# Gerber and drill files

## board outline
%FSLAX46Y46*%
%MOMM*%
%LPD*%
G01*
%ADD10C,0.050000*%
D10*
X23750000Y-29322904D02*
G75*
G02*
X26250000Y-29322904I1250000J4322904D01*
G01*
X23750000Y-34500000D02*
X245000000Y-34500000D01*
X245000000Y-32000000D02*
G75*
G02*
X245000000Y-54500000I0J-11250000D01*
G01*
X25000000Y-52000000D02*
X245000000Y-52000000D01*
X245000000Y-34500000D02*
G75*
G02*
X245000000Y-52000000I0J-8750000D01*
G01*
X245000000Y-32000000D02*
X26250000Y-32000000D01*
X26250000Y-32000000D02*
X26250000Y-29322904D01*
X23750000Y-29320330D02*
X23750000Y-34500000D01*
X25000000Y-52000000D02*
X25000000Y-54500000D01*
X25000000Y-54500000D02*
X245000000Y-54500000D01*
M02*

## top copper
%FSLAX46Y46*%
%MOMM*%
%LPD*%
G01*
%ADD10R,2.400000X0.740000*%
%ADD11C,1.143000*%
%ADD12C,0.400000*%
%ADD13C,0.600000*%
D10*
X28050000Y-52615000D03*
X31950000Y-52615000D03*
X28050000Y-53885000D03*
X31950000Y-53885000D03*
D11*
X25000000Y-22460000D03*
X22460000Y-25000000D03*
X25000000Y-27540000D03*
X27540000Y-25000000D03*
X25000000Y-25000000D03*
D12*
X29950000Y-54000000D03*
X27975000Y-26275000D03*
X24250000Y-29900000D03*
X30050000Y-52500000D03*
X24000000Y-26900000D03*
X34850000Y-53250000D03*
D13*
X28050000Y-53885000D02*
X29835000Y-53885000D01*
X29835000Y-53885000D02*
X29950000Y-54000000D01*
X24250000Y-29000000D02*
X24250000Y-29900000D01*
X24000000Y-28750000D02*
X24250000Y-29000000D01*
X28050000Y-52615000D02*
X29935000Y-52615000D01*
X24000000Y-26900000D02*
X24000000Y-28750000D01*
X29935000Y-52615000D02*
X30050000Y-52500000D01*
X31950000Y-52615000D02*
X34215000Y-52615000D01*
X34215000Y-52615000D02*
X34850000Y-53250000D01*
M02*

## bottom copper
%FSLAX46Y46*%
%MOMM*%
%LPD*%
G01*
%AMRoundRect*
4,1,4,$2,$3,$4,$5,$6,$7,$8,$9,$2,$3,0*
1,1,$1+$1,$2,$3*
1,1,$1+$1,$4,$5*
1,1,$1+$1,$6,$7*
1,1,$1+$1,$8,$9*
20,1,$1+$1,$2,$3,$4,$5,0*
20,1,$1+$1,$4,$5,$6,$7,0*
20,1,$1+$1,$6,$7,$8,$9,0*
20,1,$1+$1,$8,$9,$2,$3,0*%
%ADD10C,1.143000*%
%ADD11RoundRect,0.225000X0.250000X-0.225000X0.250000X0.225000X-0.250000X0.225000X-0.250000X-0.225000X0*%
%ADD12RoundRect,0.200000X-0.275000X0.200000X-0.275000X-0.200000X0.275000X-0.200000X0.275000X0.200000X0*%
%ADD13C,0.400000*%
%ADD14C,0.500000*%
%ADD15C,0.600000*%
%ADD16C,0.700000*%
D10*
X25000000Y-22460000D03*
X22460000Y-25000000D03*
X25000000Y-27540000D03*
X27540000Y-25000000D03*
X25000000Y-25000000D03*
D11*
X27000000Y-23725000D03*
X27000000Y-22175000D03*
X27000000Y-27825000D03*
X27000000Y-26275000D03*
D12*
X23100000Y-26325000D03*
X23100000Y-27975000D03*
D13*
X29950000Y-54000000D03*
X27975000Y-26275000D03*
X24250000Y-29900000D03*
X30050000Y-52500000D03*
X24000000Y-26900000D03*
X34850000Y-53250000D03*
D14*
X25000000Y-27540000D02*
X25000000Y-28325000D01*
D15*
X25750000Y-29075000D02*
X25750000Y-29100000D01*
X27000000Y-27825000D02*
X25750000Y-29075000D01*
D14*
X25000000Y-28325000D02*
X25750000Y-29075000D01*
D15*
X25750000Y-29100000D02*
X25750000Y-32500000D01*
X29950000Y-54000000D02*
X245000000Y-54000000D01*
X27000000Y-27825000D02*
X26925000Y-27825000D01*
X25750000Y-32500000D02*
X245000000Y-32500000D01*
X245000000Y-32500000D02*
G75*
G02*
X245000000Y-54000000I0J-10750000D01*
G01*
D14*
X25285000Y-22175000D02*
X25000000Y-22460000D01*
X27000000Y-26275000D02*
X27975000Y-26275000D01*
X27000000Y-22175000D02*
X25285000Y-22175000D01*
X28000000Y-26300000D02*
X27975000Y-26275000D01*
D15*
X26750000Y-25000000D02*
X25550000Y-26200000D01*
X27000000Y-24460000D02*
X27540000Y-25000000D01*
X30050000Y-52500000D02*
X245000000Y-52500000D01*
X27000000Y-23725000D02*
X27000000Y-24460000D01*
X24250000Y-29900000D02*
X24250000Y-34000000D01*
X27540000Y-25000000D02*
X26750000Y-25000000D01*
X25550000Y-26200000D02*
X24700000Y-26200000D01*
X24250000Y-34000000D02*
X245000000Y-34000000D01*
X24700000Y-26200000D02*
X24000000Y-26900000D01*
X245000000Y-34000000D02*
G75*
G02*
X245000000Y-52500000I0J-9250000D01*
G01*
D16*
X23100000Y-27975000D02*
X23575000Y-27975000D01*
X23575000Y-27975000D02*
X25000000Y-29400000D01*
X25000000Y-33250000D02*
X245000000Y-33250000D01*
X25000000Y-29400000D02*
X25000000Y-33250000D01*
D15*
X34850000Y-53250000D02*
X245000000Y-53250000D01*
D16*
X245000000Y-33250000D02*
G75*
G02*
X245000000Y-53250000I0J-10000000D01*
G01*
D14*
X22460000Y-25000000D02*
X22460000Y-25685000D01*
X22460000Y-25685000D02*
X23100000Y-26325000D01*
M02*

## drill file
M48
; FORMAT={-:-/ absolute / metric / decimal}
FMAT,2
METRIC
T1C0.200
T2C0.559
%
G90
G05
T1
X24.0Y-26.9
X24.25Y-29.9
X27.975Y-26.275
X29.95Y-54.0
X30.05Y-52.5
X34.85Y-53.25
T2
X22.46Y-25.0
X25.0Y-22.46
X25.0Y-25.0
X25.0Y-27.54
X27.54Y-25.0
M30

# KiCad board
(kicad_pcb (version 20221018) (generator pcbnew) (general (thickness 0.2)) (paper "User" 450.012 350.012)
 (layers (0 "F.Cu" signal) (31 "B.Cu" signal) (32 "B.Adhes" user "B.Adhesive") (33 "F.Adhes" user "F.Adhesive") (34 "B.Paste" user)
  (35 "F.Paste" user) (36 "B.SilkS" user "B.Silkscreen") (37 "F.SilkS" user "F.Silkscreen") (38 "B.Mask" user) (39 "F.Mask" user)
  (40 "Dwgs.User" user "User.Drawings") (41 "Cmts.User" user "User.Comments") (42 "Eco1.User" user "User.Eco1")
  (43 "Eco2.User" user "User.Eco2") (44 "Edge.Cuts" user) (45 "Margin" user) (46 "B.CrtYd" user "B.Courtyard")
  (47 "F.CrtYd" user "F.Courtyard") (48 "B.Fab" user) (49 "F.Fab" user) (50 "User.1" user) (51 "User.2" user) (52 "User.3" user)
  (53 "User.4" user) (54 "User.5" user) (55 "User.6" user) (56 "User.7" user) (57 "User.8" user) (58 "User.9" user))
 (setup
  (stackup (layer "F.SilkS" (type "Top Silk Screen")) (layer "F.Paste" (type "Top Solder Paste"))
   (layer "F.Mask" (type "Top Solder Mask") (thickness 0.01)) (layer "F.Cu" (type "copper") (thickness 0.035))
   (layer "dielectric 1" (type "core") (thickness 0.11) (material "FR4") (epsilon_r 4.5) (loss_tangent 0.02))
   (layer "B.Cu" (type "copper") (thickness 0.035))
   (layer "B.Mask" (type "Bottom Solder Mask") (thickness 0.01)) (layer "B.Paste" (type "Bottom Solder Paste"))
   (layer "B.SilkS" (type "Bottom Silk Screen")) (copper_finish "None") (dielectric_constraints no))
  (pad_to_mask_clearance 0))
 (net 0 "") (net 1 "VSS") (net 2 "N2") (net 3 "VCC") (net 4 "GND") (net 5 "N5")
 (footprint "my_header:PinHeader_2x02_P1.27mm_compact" (layer "F.Cu") (at 30 53.25)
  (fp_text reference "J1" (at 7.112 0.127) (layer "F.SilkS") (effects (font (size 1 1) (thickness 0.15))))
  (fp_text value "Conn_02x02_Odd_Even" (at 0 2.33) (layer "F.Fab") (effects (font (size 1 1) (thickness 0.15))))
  (pad "1" smd rect (at -1.95 -0.635) (size 2.4 0.74) (layers "F.Cu" "F.Paste" "F.Mask") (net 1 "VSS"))
  (pad "2" smd rect (at 1.95 -0.635) (size 2.4 0.74) (layers "F.Cu" "F.Paste" "F.Mask") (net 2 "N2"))
  (pad "3" smd rect (at -1.95 0.635) (size 2.4 0.74) (layers "F.Cu" "F.Paste" "F.Mask") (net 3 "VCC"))
  (pad "4" smd rect (at 1.95 0.635) (size 2.4 0.74) (layers "F.Cu" "F.Paste" "F.Mask") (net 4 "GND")))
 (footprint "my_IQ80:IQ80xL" (layer "F.Cu") (at 25 25 90)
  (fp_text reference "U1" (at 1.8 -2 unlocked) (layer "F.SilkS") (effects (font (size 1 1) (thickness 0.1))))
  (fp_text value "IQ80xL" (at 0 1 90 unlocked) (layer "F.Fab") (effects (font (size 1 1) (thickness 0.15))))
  (pad "1" thru_hole circle (at 2.54 0 90) (size 1.143 1.143) (drill 0.5588) (layers "*.Cu" "*.Mask") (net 4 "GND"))
  (pad "2" thru_hole circle (at 0 -2.54 90) (size 1.143 1.143) (drill 0.5588) (layers "*.Cu" "*.Mask") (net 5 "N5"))
  (pad "3" thru_hole circle (at -2.54 0 90) (size 1.143 1.143) (drill 0.5588) (layers "*.Cu" "*.Mask") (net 3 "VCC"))
  (pad "4" thru_hole circle (at 0 2.54 90) (size 1.143 1.143) (drill 0.5588) (layers "*.Cu" "*.Mask") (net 1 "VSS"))
  (pad "5" thru_hole circle (at 0 0 90) (size 1.143 1.143) (drill 0.5588) (layers "*.Cu" "*.Mask") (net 4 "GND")))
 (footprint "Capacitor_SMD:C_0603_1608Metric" (layer "B.Cu") (at 27 22.95 90)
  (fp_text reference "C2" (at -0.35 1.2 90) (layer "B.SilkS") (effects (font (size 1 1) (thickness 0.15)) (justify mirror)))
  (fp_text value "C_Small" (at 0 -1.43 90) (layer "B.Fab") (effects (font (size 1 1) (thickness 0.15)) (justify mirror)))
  (pad "1" smd roundrect (at -0.775 0 90) (size 0.9 0.95) (layers "B.Cu" "B.Paste" "B.Mask") (roundrect_rratio 0.25) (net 1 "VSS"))
  (pad "2" smd roundrect (at 0.775 0 90) (size 0.9 0.95) (layers "B.Cu" "B.Paste" "B.Mask") (roundrect_rratio 0.25) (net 4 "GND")))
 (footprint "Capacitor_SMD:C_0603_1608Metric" (layer "B.Cu") (at 27 27.05 90)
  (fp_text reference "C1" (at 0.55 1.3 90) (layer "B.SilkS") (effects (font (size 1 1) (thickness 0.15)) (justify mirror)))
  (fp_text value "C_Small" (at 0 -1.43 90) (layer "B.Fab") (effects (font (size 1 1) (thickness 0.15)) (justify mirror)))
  (pad "1" smd roundrect (at -0.775 0 90) (size 0.9 0.95) (layers "B.Cu" "B.Paste" "B.Mask") (roundrect_rratio 0.25) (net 3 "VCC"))
  (pad "2" smd roundrect (at 0.775 0 90) (size 0.9 0.95) (layers "B.Cu" "B.Paste" "B.Mask") (roundrect_rratio 0.25) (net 4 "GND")))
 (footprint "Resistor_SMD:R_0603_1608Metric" (layer "B.Cu") (at 23.1 27.15 -90)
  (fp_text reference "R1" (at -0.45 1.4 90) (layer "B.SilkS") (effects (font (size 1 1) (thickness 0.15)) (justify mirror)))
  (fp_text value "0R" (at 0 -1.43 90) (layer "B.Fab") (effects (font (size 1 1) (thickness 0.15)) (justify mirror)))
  (pad "1" smd roundrect (at -0.825 0 270) (size 0.8 0.95) (layers "B.Cu" "B.Paste" "B.Mask") (roundrect_rratio 0.25) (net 5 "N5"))
  (pad "2" smd roundrect (at 0.825 0 270) (size 0.8 0.95) (layers "B.Cu" "B.Paste" "B.Mask") (roundrect_rratio 0.25) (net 2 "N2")))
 (gr_arc (start 23.75 29.322904) (mid 25 20.5) (end 26.25 29.322904) (stroke (width 0.05) (type solid)) (layer "Edge.Cuts"))
 (gr_line (start 23.75 34.5) (end 245 34.5) (stroke (width 0.05) (type solid)) (layer "Edge.Cuts"))
 (gr_arc (start 245 32) (mid 256.25 43.25) (end 245 54.5) (stroke (width 0.05) (type solid)) (layer "Edge.Cuts"))
 (gr_line (start 25 52.) (end 245 52.) (stroke (width 0.05) (type solid)) (layer "Edge.Cuts"))
 (gr_arc (start 245 34.5) (mid 253.75 43.25) (end 245 52.) (stroke (width 0.05) (type solid)) (layer "Edge.Cuts"))
 (gr_line (start 245 32) (end 26.25 32) (stroke (width 0.05) (type solid)) (layer "Edge.Cuts"))
 (gr_line (start 26.25 32) (end 26.25 29.322904) (stroke (width 0.05) (type solid)) (layer "Edge.Cuts"))
 (gr_line (start 23.75 29.32033) (end 23.75 34.5) (stroke (width 0.05) (type solid)) (layer "Edge.Cuts"))
 (gr_line (start 25 52.) (end 25 54.5) (stroke (width 0.05) (type solid)) (layer "Edge.Cuts"))
 (gr_line (start 25 54.5) (end 245 54.5) (stroke (width 0.05) (type solid)) (layer "Edge.Cuts"))
 (segment (start 28.05 53.885) (end 29.835 53.885) (width 0.6) (layer "F.Cu") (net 3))
 (segment (start 29.835 53.885) (end 29.95 54.) (width 0.6) (layer "F.Cu") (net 3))
 (via (at 29.95 54.) (size 0.4) (drill 0.2) (layers "F.Cu" "B.Cu") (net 3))
 (segment (start 25 27.54) (end 25 28.325) (width 0.5) (layer "B.Cu") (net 3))
 (segment (start 25.75 29.075) (end 25.75 29.1) (width 0.6) (layer "B.Cu") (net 3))
 (segment (start 27 27.825) (end 25.75 29.075) (width 0.6) (layer "B.Cu") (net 3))
 (segment (start 25 28.325) (end 25.75 29.075) (width 0.5) (layer "B.Cu") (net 3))
 (segment (start 25.75 29.1) (end 25.75 32.5) (width 0.6) (layer "B.Cu") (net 3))
 (segment (start 29.95 54.) (end 245 54.) (width 0.6) (layer "B.Cu") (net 3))
 (segment (start 27 27.825) (end 26.925 27.825) (width 0.6) (layer "B.Cu") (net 3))
 (segment (start 25.75 32.5) (end 245 32.5) (width 0.6) (layer "B.Cu") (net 3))
 (arc (start 245 32.5) (mid 255.75 43.25) (end 245 54.) (width 0.6) (layer "B.Cu") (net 3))
 (via (at 27.975 26.275) (size 0.4) (drill 0.2) (layers "F.Cu" "B.Cu") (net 4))
 (segment (start 25.285 22.175) (end 25 22.46) (width 0.5) (layer "B.Cu") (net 4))
 (segment (start 27 26.275) (end 27.975 26.275) (width 0.5) (layer "B.Cu") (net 4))
 (segment (start 27 22.175) (end 25.285 22.175) (width 0.5) (layer "B.Cu") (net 4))
 (segment (start 28 26.3) (end 27.975 26.275) (width 0.5) (layer "B.Cu") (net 4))
 (segment (start 24.25 29) (end 24.25 29.9) (width 0.6) (layer "F.Cu") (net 1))
 (segment (start 24 28.75) (end 24.25 29) (width 0.6) (layer "F.Cu") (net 1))
 (segment (start 28.05 52.615) (end 29.935 52.615) (width 0.6) (layer "F.Cu") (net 1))
 (segment (start 24 26.9) (end 24 28.75) (width 0.6) (layer "F.Cu") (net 1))
 (segment (start 29.935 52.615) (end 30.05 52.5) (width 0.6) (layer "F.Cu") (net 1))
 (via (at 24.25 29.9) (size 0.4) (drill 0.2) (layers "F.Cu" "B.Cu") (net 1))
 (via (at 30.05 52.5) (size 0.4) (drill 0.2) (layers "F.Cu" "B.Cu") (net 1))
 (via (at 24 26.9) (size 0.4) (drill 0.2) (layers "F.Cu" "B.Cu") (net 1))
 (segment (start 26.75 25) (end 25.55 26.2) (width 0.6) (layer "B.Cu") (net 1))
 (segment (start 27 24.46) (end 27.54 25) (width 0.6) (layer "B.Cu") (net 1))
 (segment (start 30.05 52.5) (end 245 52.5) (width 0.6) (layer "B.Cu") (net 1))
 (segment (start 27 23.725) (end 27 24.46) (width 0.6) (layer "B.Cu") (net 1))
 (segment (start 24.25 29.9) (end 24.25 34) (width 0.6) (layer "B.Cu") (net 1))
 (segment (start 27.54 25) (end 26.75 25) (width 0.6) (layer "B.Cu") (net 1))
 (segment (start 25.55 26.2) (end 24.7 26.2) (width 0.6) (layer "B.Cu") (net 1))
 (segment (start 24.25 34) (end 245 34) (width 0.6) (layer "B.Cu") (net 1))
 (segment (start 24.7 26.2) (end 24 26.9) (width 0.6) (layer "B.Cu") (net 1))
 (arc (start 245 34) (mid 254.25 43.25) (end 245 52.5) (width 0.6) (layer "B.Cu") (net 1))
 (segment (start 31.95 52.615) (end 34.215 52.615) (width 0.6) (layer "F.Cu") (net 2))
 (segment (start 34.215 52.615) (end 34.85 53.25) (width 0.6) (layer "F.Cu") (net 2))
 (via (at 34.85 53.25) (size 0.4) (drill 0.2) (layers "F.Cu" "B.Cu") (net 2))
 (segment (start 23.1 27.975) (end 23.575 27.975) (width 0.7) (layer "B.Cu") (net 2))
 (segment (start 23.575 27.975) (end 25 29.4) (width 0.7) (layer "B.Cu") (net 2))
 (segment (start 25 33.25) (end 245 33.25) (width 0.7) (layer "B.Cu") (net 2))
 (segment (start 25 29.4) (end 25 33.25) (width 0.7) (layer "B.Cu") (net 2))
 (segment (start 34.85 53.25) (end 245 53.25) (width 0.6) (layer "B.Cu") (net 2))
 (arc (start 245 33.25) (mid 255. 43.25) (end 245 53.25) (width 0.7) (layer "B.Cu") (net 2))
 (segment (start 22.46 25) (end 22.46 25.685) (width 0.5) (layer "B.Cu") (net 5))
 (segment (start 22.46 25.685) (end 23.1 26.325) (width 0.5) (layer "B.Cu") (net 5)))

